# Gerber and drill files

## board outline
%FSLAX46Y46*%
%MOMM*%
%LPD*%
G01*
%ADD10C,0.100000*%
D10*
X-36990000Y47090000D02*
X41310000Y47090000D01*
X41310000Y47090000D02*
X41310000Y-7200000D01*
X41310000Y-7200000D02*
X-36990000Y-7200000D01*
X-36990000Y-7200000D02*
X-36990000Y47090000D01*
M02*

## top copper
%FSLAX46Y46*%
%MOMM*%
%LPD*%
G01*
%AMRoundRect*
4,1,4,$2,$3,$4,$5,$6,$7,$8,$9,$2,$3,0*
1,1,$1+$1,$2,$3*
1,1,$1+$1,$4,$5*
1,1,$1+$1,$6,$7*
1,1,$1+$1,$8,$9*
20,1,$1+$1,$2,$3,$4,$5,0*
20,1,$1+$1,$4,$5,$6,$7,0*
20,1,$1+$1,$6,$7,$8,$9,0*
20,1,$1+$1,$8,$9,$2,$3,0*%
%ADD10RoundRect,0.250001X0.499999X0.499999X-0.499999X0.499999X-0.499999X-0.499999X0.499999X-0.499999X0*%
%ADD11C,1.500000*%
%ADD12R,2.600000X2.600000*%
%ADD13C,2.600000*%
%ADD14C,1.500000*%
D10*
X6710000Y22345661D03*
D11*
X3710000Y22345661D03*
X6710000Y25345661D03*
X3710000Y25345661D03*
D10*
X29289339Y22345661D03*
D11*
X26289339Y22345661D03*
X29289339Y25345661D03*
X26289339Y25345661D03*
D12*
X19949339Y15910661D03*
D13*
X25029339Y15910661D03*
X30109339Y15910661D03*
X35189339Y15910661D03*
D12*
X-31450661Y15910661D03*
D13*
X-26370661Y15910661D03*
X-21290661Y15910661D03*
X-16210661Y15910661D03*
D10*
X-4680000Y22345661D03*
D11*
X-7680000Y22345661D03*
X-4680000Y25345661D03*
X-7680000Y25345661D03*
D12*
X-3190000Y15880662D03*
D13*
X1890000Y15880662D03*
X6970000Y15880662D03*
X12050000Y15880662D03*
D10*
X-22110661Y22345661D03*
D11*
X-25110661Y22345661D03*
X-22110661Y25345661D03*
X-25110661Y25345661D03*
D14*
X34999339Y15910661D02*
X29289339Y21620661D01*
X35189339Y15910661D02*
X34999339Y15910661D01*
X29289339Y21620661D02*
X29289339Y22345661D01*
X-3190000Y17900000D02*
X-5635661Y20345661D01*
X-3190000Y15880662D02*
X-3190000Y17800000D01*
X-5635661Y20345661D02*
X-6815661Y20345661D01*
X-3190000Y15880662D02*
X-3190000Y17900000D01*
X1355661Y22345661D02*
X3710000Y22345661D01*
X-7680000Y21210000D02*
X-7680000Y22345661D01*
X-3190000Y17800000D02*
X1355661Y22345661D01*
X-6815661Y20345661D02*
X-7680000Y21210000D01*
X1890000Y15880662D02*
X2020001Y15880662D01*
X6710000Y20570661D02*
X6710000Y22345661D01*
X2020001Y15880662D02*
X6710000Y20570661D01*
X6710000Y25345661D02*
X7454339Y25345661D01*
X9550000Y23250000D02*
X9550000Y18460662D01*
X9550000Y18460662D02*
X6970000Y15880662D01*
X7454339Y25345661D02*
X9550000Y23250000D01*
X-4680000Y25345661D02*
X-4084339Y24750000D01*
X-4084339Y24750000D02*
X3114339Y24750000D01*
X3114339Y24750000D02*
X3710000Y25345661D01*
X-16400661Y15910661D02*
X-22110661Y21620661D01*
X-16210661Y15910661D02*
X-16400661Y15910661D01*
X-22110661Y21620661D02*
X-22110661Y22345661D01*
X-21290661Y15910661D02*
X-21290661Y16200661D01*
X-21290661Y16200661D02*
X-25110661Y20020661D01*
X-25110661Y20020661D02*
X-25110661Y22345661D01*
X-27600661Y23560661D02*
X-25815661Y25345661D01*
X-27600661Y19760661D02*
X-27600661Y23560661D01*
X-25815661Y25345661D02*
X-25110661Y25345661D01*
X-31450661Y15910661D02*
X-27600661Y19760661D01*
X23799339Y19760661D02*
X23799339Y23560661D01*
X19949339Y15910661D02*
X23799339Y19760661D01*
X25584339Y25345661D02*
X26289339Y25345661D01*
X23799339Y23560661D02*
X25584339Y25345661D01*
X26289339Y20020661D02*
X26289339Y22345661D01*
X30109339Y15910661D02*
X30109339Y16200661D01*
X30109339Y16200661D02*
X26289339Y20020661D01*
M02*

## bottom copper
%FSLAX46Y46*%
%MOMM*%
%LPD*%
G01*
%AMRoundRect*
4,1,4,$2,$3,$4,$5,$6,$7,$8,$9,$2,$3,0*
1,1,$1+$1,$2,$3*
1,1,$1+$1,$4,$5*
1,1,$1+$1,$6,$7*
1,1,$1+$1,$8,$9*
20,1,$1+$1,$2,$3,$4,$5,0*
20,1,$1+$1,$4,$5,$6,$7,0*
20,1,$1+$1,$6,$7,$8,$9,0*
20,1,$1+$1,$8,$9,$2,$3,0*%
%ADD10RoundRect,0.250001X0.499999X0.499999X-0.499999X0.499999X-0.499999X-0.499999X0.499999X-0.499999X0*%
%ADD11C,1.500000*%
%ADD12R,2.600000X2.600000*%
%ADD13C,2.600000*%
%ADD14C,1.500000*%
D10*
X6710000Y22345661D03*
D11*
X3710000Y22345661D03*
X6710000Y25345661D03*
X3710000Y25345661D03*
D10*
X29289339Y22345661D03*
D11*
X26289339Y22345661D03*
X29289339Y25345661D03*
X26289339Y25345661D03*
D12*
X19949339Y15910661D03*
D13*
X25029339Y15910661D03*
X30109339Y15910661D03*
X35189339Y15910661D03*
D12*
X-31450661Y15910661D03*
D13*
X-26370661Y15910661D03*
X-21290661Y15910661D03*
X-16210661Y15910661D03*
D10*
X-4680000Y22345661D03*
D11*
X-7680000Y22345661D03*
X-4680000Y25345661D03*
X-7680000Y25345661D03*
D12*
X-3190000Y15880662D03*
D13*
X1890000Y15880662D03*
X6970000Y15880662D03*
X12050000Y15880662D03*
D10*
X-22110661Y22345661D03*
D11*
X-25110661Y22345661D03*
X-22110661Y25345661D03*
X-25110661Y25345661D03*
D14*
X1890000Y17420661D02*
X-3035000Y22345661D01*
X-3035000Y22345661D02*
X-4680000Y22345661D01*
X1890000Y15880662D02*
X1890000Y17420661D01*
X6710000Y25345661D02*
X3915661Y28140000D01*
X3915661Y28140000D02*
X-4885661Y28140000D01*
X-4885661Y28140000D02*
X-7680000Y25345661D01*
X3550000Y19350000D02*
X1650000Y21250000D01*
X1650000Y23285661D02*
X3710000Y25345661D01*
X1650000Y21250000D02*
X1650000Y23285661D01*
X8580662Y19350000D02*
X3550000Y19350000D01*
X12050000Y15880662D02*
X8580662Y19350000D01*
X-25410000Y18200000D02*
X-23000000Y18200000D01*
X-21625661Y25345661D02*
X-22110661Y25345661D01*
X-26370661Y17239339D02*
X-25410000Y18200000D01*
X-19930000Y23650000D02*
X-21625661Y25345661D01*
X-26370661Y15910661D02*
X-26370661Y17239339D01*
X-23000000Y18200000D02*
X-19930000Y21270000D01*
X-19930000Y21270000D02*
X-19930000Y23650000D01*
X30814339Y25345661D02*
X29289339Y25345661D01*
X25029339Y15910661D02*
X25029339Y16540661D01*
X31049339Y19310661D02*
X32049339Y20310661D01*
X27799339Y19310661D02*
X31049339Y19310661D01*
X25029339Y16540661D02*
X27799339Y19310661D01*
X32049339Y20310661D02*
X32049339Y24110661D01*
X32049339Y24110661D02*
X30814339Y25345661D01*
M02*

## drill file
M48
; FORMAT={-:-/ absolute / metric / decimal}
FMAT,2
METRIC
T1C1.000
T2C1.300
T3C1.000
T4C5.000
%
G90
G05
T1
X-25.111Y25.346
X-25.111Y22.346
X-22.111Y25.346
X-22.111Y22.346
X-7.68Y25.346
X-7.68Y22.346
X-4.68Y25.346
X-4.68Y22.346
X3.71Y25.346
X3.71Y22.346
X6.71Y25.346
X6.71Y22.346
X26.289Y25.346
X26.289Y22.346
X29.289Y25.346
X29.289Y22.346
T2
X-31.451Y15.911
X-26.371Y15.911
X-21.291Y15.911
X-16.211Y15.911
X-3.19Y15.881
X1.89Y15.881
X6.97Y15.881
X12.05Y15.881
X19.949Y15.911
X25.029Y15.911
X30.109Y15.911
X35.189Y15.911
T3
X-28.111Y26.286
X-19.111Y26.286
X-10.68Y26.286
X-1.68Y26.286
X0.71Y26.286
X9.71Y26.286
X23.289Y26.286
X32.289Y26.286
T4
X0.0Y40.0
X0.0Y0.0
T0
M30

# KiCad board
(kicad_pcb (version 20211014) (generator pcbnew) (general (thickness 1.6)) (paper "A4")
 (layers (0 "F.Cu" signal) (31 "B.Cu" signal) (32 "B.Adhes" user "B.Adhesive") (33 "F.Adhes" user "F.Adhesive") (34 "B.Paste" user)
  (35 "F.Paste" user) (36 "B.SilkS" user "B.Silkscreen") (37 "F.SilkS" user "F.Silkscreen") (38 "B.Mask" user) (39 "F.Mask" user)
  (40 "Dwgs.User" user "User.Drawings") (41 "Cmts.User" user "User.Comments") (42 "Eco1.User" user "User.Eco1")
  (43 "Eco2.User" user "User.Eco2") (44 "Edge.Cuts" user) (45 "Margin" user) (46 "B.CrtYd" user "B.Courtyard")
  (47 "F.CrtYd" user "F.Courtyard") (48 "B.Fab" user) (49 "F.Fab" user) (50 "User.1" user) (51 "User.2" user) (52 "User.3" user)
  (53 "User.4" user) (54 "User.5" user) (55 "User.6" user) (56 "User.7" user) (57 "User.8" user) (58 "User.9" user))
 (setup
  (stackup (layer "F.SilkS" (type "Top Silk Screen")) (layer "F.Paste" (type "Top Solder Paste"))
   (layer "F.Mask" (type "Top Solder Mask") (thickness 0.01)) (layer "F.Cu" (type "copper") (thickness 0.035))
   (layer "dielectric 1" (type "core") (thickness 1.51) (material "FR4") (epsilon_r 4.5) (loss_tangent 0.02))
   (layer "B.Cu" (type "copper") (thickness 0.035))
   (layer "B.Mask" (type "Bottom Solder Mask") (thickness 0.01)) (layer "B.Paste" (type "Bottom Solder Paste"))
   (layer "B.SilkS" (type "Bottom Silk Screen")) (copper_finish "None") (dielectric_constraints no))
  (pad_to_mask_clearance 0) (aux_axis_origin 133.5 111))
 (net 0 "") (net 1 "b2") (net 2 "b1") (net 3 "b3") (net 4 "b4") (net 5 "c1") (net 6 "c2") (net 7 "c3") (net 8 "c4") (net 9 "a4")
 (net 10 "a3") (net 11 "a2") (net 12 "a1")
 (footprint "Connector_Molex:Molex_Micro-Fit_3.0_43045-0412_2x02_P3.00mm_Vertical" (layer "F.Cu") (at 140.21 88.654339 180)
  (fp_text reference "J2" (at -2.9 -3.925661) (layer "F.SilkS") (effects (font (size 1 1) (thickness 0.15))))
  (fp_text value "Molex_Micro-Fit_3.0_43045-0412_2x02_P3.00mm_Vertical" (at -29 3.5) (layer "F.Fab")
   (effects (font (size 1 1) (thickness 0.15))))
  (pad "" np_thru_hole circle (at 6 3.94 180) (size 1 1) (drill 1) (layers F&B.Cu *.Mask))
  (pad "" np_thru_hole circle (at -3 3.94 180) (size 1 1) (drill 1) (layers F&B.Cu *.Mask))
  (pad "1" thru_hole roundrect (at 0 0 180) (size 1.5 1.5) (drill 1) (layers *.Cu *.Mask) (roundrect_rratio 0.1666673333) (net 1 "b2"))
  (pad "2" thru_hole circle (at 3 0 180) (size 1.5 1.5) (drill 1) (layers *.Cu *.Mask) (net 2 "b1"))
  (pad "3" thru_hole circle (at 0 3 180) (size 1.5 1.5) (drill 1) (layers *.Cu *.Mask) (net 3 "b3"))
  (pad "4" thru_hole circle (at 3 3 180) (size 1.5 1.5) (drill 1) (layers *.Cu *.Mask) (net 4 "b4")))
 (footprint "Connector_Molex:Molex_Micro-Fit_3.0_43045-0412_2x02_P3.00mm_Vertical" (layer "F.Cu") (at 162.789339 88.654339 180)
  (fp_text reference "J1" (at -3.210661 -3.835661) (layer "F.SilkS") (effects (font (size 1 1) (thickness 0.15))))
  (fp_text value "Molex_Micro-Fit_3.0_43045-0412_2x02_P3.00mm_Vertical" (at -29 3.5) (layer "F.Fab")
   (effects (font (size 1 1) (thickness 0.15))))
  (pad "" np_thru_hole circle (at -3 3.94 180) (size 1 1) (drill 1) (layers F&B.Cu *.Mask))
  (pad "" np_thru_hole circle (at 6 3.94 180) (size 1 1) (drill 1) (layers F&B.Cu *.Mask))
  (pad "1" thru_hole roundrect (at 0 0 180) (size 1.5 1.5) (drill 1) (layers *.Cu *.Mask) (roundrect_rratio 0.1666673333) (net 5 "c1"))
  (pad "2" thru_hole circle (at 3 0 180) (size 1.5 1.5) (drill 1) (layers *.Cu *.Mask) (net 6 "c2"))
  (pad "3" thru_hole circle (at 0 3 180) (size 1.5 1.5) (drill 1) (layers *.Cu *.Mask) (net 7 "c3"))
  (pad "4" thru_hole circle (at 3 3 180) (size 1.5 1.5) (drill 1) (layers *.Cu *.Mask) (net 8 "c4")))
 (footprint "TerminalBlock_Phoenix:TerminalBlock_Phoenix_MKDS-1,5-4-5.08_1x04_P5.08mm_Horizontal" (layer "F.Cu") (at 153.449339 95.089339)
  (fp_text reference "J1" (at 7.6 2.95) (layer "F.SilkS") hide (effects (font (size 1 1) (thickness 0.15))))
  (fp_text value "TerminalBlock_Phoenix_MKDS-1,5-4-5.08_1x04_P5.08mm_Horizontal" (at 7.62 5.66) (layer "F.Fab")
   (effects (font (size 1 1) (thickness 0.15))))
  (pad "1" thru_hole rect (at 0 0) (size 2.6 2.6) (drill 1.3) (layers *.Cu *.Mask) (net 8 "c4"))
  (pad "2" thru_hole circle (at 5.08 0) (size 2.6 2.6) (drill 1.3) (layers *.Cu *.Mask) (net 7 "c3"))
  (pad "3" thru_hole circle (at 10.16 0) (size 2.6 2.6) (drill 1.3) (layers *.Cu *.Mask) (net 6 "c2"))
  (pad "4" thru_hole circle (at 15.24 0) (size 2.6 2.6) (drill 1.3) (layers *.Cu *.Mask) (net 5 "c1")))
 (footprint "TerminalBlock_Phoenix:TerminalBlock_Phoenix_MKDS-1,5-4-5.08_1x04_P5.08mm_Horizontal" (layer "F.Cu") (at 102.049339 95.089339)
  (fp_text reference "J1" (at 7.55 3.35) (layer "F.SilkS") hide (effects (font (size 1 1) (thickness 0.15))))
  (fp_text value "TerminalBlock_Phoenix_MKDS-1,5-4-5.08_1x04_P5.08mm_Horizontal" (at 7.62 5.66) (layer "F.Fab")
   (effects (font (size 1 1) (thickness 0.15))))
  (pad "1" thru_hole rect (at 0 0) (size 2.6 2.6) (drill 1.3) (layers *.Cu *.Mask) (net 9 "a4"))
  (pad "2" thru_hole circle (at 5.08 0) (size 2.6 2.6) (drill 1.3) (layers *.Cu *.Mask) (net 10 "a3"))
  (pad "3" thru_hole circle (at 10.16 0) (size 2.6 2.6) (drill 1.3) (layers *.Cu *.Mask) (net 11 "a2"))
  (pad "4" thru_hole circle (at 15.24 0) (size 2.6 2.6) (drill 1.3) (layers *.Cu *.Mask) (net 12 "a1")))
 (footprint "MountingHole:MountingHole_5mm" (layer "F.Cu") (at 133.5 71)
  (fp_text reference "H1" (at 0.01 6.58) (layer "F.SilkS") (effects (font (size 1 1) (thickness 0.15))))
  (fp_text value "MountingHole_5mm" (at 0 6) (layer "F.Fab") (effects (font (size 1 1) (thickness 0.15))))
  (pad "" np_thru_hole circle (at 0 0) (size 5 5) (drill 5) (layers F&B.Cu *.Mask)))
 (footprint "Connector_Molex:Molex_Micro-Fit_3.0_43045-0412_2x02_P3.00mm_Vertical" (layer "F.Cu") (at 128.82 88.654339 180)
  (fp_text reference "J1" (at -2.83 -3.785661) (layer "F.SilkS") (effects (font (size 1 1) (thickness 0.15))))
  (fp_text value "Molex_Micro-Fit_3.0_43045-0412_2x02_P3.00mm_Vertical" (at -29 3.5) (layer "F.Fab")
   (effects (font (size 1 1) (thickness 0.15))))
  (pad "" np_thru_hole circle (at -3 3.94 180) (size 1 1) (drill 1) (layers F&B.Cu *.Mask))
  (pad "" np_thru_hole circle (at 6 3.94 180) (size 1 1) (drill 1) (layers F&B.Cu *.Mask))
  (pad "1" thru_hole roundrect (at 0 0 180) (size 1.5 1.5) (drill 1) (layers *.Cu *.Mask) (roundrect_rratio 0.1666673333) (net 1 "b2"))
  (pad "2" thru_hole circle (at 3 0 180) (size 1.5 1.5) (drill 1) (layers *.Cu *.Mask) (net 2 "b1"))
  (pad "3" thru_hole circle (at 0 3 180) (size 1.5 1.5) (drill 1) (layers *.Cu *.Mask) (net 4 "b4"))
  (pad "4" thru_hole circle (at 3 3 180) (size 1.5 1.5) (drill 1) (layers *.Cu *.Mask) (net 3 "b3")))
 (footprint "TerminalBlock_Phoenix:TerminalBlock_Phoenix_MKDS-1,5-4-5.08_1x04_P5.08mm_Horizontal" (layer "F.Cu") (at 130.31 95.119338)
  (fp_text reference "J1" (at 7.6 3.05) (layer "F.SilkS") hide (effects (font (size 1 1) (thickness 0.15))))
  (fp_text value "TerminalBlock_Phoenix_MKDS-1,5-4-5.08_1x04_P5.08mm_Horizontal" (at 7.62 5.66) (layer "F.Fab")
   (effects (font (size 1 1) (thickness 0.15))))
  (pad "1" thru_hole rect (at 0 0) (size 2.6 2.6) (drill 1.3) (layers *.Cu *.Mask) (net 2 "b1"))
  (pad "2" thru_hole circle (at 5.08 0) (size 2.6 2.6) (drill 1.3) (layers *.Cu *.Mask) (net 1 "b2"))
  (pad "3" thru_hole circle (at 10.16 0) (size 2.6 2.6) (drill 1.3) (layers *.Cu *.Mask) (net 3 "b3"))
  (pad "4" thru_hole circle (at 15.24 0) (size 2.6 2.6) (drill 1.3) (layers *.Cu *.Mask) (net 4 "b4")))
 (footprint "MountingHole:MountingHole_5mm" (layer "F.Cu") (at 133.5 111)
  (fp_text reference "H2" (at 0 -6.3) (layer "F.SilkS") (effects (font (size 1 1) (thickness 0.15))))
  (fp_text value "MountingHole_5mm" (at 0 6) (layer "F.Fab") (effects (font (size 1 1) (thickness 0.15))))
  (pad "" np_thru_hole circle (at 0 0) (size 5 5) (drill 5) (layers *.Cu *.Mask)))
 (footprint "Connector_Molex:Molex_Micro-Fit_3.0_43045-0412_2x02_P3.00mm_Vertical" (layer "F.Cu") (at 111.389339 88.654339 180)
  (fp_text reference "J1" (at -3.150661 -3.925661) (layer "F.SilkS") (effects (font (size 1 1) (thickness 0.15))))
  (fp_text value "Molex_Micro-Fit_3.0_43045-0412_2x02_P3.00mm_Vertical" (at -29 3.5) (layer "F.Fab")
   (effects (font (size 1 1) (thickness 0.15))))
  (pad "" np_thru_hole circle (at -3 3.94 180) (size 1 1) (drill 1) (layers *.Cu *.Mask))
  (pad "" np_thru_hole circle (at 6 3.94 180) (size 1 1) (drill 1) (layers *.Cu *.Mask))
  (pad "1" thru_hole roundrect (at 0 0 180) (size 1.5 1.5) (drill 1) (layers *.Cu *.Mask) (roundrect_rratio 0.1666673333) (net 12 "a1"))
  (pad "2" thru_hole circle (at 3 0 180) (size 1.5 1.5) (drill 1) (layers *.Cu *.Mask) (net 11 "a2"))
  (pad "3" thru_hole circle (at 0 3 180) (size 1.5 1.5) (drill 1) (layers *.Cu *.Mask) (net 10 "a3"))
  (pad "4" thru_hole circle (at 3 3 180) (size 1.5 1.5) (drill 1) (layers *.Cu *.Mask) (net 9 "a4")))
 (gr_rect (start 96.51 63.91) (end 174.81 118.2) (layer "Edge.Cuts") (width 0.1) (fill none))
 (segment (start 168.499339 95.089339) (end 162.789339 89.379339) (width 1.5) (layer "F.Cu") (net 5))
 (segment (start 168.689339 95.089339) (end 168.499339 95.089339) (width 1.5) (layer "F.Cu") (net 5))
 (segment (start 162.789339 89.379339) (end 162.789339 88.654339) (width 1.5) (layer "F.Cu") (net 5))
 (segment (start 130.31 93.1) (end 127.864339 90.654339) (width 1.5) (layer "F.Cu") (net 2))
 (segment (start 130.31 95.119338) (end 130.31 93.2) (width 1.5) (layer "F.Cu") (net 2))
 (segment (start 127.864339 90.654339) (end 126.684339 90.654339) (width 1.5) (layer "F.Cu") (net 2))
 (segment (start 130.31 95.119338) (end 130.31 93.1) (width 1.5) (layer "F.Cu") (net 2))
 (segment (start 134.855661 88.654339) (end 137.21 88.654339) (width 1.5) (layer "F.Cu") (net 2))
 (segment (start 125.82 89.79) (end 125.82 88.654339) (width 1.5) (layer "F.Cu") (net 2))
 (segment (start 130.31 93.2) (end 134.855661 88.654339) (width 1.5) (layer "F.Cu") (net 2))
 (segment (start 126.684339 90.654339) (end 125.82 89.79) (width 1.5) (layer "F.Cu") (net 2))
 (segment (start 135.39 95.119338) (end 135.520001 95.119338) (width 1.5) (layer "F.Cu") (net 1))
 (segment (start 140.21 90.429339) (end 140.21 88.654339) (width 1.5) (layer "F.Cu") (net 1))
 (segment (start 135.520001 95.119338) (end 140.21 90.429339) (width 1.5) (layer "F.Cu") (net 1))
 (segment (start 135.39 93.579339) (end 130.465 88.654339) (width 1.5) (layer "B.Cu") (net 1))
 (segment (start 130.465 88.654339) (end 128.82 88.654339) (width 1.5) (layer "B.Cu") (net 1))
 (segment (start 135.39 95.119338) (end 135.39 93.579339) (width 1.5) (layer "B.Cu") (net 1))
 (segment (start 140.21 85.654339) (end 140.954339 85.654339) (width 1.5) (layer "F.Cu") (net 3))
 (segment (start 143.05 87.75) (end 143.05 92.539338) (width 1.5) (layer "F.Cu") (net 3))
 (segment (start 143.05 92.539338) (end 140.47 95.119338) (width 1.5) (layer "F.Cu") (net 3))
 (segment (start 140.954339 85.654339) (end 143.05 87.75) (width 1.5) (layer "F.Cu") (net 3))
 (segment (start 140.21 85.654339) (end 137.415661 82.86) (width 1.5) (layer "B.Cu") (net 3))
 (segment (start 137.415661 82.86) (end 128.614339 82.86) (width 1.5) (layer "B.Cu") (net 3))
 (segment (start 128.614339 82.86) (end 125.82 85.654339) (width 1.5) (layer "B.Cu") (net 3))
 (segment (start 128.82 85.654339) (end 129.415661 86.25) (width 1.5) (layer "F.Cu") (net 4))
 (segment (start 129.415661 86.25) (end 136.614339 86.25) (width 1.5) (layer "F.Cu") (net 4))
 (segment (start 136.614339 86.25) (end 137.21 85.654339) (width 1.5) (layer "F.Cu") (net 4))
 (segment (start 137.05 91.65) (end 135.15 89.75) (width 1.5) (layer "B.Cu") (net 4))
 (segment (start 135.15 87.714339) (end 137.21 85.654339) (width 1.5) (layer "B.Cu") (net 4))
 (segment (start 135.15 89.75) (end 135.15 87.714339) (width 1.5) (layer "B.Cu") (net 4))
 (segment (start 142.080662 91.65) (end 137.05 91.65) (width 1.5) (layer "B.Cu") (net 4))
 (segment (start 145.55 95.119338) (end 142.080662 91.65) (width 1.5) (layer "B.Cu") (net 4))
 (segment (start 117.099339 95.089339) (end 111.389339 89.379339) (width 1.5) (layer "F.Cu") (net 12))
 (segment (start 117.289339 95.089339) (end 117.099339 95.089339) (width 1.5) (layer "F.Cu") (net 12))
 (segment (start 111.389339 89.379339) (end 111.389339 88.654339) (width 1.5) (layer "F.Cu") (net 12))
 (segment (start 112.209339 95.089339) (end 112.209339 94.799339) (width 1.5) (layer "F.Cu") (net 11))
 (segment (start 112.209339 94.799339) (end 108.389339 90.979339) (width 1.5) (layer "F.Cu") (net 11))
 (segment (start 108.389339 90.979339) (end 108.389339 88.654339) (width 1.5) (layer "F.Cu") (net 11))
 (segment (start 108.09 92.8) (end 110.5 92.8) (width 1.5) (layer "B.Cu") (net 10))
 (segment (start 111.874339 85.654339) (end 111.389339 85.654339) (width 1.5) (layer "B.Cu") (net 10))
 (segment (start 107.129339 93.760661) (end 108.09 92.8) (width 1.5) (layer "B.Cu") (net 10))
 (segment (start 113.57 87.35) (end 111.874339 85.654339) (width 1.5) (layer "B.Cu") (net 10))
 (segment (start 107.129339 95.089339) (end 107.129339 93.760661) (width 1.5) (layer "B.Cu") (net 10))
 (segment (start 110.5 92.8) (end 113.57 89.73) (width 1.5) (layer "B.Cu") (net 10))
 (segment (start 113.57 89.73) (end 113.57 87.35) (width 1.5) (layer "B.Cu") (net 10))
 (segment (start 105.899339 87.439339) (end 107.684339 85.654339) (width 1.5) (layer "F.Cu") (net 9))
 (segment (start 105.899339 91.239339) (end 105.899339 87.439339) (width 1.5) (layer "F.Cu") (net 9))
 (segment (start 107.684339 85.654339) (end 108.389339 85.654339) (width 1.5) (layer "F.Cu") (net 9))
 (segment (start 102.049339 95.089339) (end 105.899339 91.239339) (width 1.5) (layer "F.Cu") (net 9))
 (segment (start 157.299339 91.239339) (end 157.299339 87.439339) (width 1.5) (layer "F.Cu") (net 8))
 (segment (start 153.449339 95.089339) (end 157.299339 91.239339) (width 1.5) (layer "F.Cu") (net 8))
 (segment (start 159.084339 85.654339) (end 159.789339 85.654339) (width 1.5) (layer "F.Cu") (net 8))
 (segment (start 157.299339 87.439339) (end 159.084339 85.654339) (width 1.5) (layer "F.Cu") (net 8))
 (segment (start 164.314339 85.654339) (end 162.789339 85.654339) (width 1.5) (layer "B.Cu") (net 7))
 (segment (start 158.529339 95.089339) (end 158.529339 94.459339) (width 1.5) (layer "B.Cu") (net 7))
 (segment (start 164.549339 91.689339) (end 165.549339 90.689339) (width 1.5) (layer "B.Cu") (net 7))
 (segment (start 161.299339 91.689339) (end 164.549339 91.689339) (width 1.5) (layer "B.Cu") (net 7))
 (segment (start 158.529339 94.459339) (end 161.299339 91.689339) (width 1.5) (layer "B.Cu") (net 7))
 (segment (start 165.549339 90.689339) (end 165.549339 86.889339) (width 1.5) (layer "B.Cu") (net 7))
 (segment (start 165.549339 86.889339) (end 164.314339 85.654339) (width 1.5) (layer "B.Cu") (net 7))
 (segment (start 159.789339 90.979339) (end 159.789339 88.654339) (width 1.5) (layer "F.Cu") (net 6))
 (segment (start 163.609339 95.089339) (end 163.609339 94.799339) (width 1.5) (layer "F.Cu") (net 6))
 (segment (start 163.609339 94.799339) (end 159.789339 90.979339) (width 1.5) (layer "F.Cu") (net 6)))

